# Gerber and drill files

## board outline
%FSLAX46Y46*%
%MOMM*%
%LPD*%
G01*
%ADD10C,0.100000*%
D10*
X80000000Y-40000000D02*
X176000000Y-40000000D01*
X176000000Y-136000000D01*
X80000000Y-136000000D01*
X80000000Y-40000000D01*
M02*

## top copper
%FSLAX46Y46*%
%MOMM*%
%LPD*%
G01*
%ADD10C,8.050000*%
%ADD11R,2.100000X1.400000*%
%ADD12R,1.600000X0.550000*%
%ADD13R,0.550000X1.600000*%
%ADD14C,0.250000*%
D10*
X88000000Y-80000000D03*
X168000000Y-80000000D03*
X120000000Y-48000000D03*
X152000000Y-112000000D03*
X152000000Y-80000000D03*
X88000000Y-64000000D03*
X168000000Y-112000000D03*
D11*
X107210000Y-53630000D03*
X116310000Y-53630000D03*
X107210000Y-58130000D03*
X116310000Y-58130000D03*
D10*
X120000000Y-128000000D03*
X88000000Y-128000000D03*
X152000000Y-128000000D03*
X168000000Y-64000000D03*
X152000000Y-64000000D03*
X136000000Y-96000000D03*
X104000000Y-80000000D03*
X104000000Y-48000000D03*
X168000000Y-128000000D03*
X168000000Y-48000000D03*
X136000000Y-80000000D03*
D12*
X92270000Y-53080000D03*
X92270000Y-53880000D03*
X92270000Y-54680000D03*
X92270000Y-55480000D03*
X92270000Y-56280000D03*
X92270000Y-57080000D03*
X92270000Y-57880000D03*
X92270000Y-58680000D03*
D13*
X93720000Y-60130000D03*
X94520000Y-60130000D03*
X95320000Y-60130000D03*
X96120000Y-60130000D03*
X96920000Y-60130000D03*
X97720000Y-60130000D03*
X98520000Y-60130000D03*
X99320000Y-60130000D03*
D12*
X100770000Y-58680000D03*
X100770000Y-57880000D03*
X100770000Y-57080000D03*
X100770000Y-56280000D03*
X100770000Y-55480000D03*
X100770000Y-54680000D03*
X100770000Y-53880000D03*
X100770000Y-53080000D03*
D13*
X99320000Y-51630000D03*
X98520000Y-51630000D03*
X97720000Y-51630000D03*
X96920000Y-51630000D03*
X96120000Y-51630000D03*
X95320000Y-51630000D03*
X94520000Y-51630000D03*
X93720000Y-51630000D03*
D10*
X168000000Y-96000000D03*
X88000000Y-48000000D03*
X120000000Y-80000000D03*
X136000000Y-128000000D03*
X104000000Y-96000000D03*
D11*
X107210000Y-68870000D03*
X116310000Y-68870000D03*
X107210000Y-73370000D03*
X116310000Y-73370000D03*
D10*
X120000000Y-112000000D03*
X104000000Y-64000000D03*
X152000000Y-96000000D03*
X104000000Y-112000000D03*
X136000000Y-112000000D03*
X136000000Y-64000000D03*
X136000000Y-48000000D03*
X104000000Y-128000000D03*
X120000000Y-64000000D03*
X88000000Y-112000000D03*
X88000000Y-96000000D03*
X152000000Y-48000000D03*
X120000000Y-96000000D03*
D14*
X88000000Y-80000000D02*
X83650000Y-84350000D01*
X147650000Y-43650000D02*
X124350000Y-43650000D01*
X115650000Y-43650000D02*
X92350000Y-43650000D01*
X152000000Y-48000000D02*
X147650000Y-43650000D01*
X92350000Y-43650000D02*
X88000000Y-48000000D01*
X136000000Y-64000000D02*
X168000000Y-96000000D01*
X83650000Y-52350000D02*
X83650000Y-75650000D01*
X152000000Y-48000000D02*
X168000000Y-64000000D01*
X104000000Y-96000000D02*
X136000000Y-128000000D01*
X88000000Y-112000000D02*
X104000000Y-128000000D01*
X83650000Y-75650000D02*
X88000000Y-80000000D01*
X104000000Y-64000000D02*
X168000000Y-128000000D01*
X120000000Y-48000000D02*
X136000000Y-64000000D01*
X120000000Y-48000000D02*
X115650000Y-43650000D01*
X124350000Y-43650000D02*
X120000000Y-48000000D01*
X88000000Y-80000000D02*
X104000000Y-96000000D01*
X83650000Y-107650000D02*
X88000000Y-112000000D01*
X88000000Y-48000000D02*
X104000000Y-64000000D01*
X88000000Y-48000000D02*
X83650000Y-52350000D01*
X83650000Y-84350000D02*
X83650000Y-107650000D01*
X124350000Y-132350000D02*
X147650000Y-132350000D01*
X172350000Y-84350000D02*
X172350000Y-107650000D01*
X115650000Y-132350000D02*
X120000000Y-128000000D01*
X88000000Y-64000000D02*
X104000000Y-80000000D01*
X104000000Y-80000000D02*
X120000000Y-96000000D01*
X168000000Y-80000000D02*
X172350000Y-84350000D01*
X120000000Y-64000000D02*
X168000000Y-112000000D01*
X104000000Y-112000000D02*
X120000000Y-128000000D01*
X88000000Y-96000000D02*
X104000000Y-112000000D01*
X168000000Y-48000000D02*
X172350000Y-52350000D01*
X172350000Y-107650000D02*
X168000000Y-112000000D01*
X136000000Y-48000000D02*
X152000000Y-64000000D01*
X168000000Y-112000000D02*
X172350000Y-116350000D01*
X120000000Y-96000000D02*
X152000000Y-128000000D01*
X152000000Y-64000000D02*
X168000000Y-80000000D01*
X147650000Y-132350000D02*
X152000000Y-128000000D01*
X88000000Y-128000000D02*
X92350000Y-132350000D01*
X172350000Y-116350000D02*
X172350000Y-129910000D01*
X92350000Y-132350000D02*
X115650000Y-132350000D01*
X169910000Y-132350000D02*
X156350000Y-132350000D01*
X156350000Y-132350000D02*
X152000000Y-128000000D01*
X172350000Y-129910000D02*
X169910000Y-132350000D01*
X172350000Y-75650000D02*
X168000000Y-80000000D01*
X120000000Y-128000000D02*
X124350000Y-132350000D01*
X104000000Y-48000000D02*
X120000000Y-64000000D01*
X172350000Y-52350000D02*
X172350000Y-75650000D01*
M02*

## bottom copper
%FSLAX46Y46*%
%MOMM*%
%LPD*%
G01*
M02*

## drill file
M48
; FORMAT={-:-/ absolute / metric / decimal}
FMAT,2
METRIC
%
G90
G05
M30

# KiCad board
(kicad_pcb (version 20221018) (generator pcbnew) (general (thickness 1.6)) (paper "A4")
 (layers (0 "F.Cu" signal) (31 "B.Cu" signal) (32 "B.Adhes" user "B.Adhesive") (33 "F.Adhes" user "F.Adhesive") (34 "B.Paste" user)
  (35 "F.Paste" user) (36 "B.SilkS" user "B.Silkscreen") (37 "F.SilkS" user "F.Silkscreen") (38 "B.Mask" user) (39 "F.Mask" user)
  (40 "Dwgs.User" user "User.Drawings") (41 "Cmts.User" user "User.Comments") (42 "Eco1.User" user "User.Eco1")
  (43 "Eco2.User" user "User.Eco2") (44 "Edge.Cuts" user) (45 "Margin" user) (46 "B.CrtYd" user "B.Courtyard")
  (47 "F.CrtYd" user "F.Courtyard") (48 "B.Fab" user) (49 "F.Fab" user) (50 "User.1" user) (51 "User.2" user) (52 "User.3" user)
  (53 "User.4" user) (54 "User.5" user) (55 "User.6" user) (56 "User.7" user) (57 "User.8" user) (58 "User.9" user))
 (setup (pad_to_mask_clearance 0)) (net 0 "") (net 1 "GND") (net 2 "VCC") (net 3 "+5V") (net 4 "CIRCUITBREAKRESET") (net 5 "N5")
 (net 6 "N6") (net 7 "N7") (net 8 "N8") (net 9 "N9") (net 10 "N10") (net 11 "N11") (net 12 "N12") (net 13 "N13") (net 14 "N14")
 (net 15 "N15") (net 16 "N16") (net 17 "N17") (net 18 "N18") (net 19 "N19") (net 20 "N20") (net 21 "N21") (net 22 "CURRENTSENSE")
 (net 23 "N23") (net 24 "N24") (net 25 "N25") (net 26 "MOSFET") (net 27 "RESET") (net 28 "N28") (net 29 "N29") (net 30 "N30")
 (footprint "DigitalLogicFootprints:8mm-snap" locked (layer "F.Cu") (at 88 80)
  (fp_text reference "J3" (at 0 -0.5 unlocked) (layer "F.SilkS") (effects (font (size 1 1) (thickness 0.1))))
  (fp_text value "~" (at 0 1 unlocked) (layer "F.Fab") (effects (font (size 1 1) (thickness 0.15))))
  (pad "1" smd circle locked (at 0 0) (size 8.05 8.05) (layers "F.Cu" "F.Paste" "F.Mask") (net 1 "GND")))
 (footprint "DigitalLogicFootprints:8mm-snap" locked (layer "F.Cu") (at 168 80)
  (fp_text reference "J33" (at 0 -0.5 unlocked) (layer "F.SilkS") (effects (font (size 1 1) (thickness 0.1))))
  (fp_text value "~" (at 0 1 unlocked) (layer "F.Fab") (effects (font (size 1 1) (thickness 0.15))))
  (pad "1" smd circle locked (at 0 0) (size 8.05 8.05) (layers "F.Cu" "F.Paste" "F.Mask") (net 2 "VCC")))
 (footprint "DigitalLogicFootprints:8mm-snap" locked (layer "F.Cu") (at 120 48)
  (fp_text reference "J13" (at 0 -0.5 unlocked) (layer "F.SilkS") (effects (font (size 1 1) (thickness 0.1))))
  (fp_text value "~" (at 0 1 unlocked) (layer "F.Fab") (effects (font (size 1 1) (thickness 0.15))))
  (pad "1" smd circle locked (at 0 0) (size 8.05 8.05) (layers "F.Cu" "F.Paste" "F.Mask") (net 1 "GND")))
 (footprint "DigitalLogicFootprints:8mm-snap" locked (layer "F.Cu") (at 152 112)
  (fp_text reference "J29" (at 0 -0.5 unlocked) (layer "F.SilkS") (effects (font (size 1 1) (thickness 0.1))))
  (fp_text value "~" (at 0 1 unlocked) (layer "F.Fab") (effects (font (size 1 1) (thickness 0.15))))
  (pad "1" smd circle locked (at 0 0) (size 8.05 8.05) (layers "F.Cu" "F.Paste" "F.Mask") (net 1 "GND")))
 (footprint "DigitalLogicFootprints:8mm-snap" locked (layer "F.Cu") (at 152 80)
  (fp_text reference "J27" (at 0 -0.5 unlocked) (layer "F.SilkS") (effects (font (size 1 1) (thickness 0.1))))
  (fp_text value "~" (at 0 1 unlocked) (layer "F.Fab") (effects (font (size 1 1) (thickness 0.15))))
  (pad "1" smd circle locked (at 0 0) (size 8.05 8.05) (layers "F.Cu" "F.Paste" "F.Mask") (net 1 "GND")))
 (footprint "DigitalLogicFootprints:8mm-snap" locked (layer "F.Cu") (at 88 64)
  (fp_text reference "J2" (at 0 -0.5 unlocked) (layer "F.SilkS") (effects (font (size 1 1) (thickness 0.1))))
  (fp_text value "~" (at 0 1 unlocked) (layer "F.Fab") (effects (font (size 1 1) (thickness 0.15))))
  (pad "1" smd circle locked (at 0 0) (size 8.05 8.05) (layers "F.Cu" "F.Paste" "F.Mask") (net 2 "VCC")))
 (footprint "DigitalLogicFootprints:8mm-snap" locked (layer "F.Cu") (at 168 112)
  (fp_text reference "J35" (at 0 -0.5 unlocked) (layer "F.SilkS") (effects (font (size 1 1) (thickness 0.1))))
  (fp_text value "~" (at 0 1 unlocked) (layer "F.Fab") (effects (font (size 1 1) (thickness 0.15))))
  (pad "1" smd circle locked (at 0 0) (size 8.05 8.05) (layers "F.Cu" "F.Paste" "F.Mask") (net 2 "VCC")))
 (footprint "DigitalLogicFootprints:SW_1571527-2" (layer "F.Cu") (at 111.76 55.88)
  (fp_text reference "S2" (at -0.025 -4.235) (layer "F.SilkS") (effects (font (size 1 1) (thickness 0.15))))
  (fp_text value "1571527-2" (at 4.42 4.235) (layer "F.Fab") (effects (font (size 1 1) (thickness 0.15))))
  (pad "1" smd rect (at -4.55 -2.25) (size 2.1 1.4) (layers "F.Cu" "F.Paste" "F.Mask") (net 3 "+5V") (solder_mask_margin 0.102))
  (pad "2" smd rect (at 4.55 -2.25) (size 2.1 1.4) (layers "F.Cu" "F.Paste" "F.Mask") (solder_mask_margin 0.102))
  (pad "3" smd rect (at -4.55 2.25) (size 2.1 1.4) (layers "F.Cu" "F.Paste" "F.Mask") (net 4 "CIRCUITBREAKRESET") (solder_mask_margin 0.102))
  (pad "4" smd rect (at 4.55 2.25) (size 2.1 1.4) (layers "F.Cu" "F.Paste" "F.Mask") (solder_mask_margin 0.102)))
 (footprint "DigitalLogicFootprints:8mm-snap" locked (layer "F.Cu") (at 120 128)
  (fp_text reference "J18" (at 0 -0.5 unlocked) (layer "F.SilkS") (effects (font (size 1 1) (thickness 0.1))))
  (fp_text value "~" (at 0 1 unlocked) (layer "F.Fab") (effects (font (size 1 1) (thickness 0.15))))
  (pad "1" smd circle locked (at 0 0) (size 8.05 8.05) (layers "F.Cu" "F.Paste" "F.Mask") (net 2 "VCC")))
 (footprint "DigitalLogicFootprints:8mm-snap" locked (layer "F.Cu") (at 88 128)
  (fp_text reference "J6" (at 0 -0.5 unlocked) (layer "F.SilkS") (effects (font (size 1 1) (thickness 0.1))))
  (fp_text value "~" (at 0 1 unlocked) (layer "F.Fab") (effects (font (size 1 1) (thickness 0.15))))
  (pad "1" smd circle locked (at 0 0) (size 8.05 8.05) (layers "F.Cu" "F.Paste" "F.Mask") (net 2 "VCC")))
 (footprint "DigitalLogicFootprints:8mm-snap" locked (layer "F.Cu") (at 152 128)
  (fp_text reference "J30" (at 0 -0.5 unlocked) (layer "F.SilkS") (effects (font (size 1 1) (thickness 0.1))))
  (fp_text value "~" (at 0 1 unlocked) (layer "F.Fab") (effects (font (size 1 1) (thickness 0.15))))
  (pad "1" smd circle locked (at 0 0) (size 8.05 8.05) (layers "F.Cu" "F.Paste" "F.Mask") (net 2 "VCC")))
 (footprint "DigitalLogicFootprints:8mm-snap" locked (layer "F.Cu") (at 168 64)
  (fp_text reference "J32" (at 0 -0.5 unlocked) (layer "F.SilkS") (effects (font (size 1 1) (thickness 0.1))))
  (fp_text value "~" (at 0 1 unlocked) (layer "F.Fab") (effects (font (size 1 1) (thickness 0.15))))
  (pad "1" smd circle locked (at 0 0) (size 8.05 8.05) (layers "F.Cu" "F.Paste" "F.Mask") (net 1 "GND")))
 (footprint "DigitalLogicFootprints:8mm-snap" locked (layer "F.Cu") (at 152 64)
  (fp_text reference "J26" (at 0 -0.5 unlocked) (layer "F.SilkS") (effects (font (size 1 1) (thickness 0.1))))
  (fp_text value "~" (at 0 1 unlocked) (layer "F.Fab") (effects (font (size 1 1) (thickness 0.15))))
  (pad "1" smd circle locked (at 0 0) (size 8.05 8.05) (layers "F.Cu" "F.Paste" "F.Mask") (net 2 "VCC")))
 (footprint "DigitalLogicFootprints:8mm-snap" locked (layer "F.Cu") (at 136 96)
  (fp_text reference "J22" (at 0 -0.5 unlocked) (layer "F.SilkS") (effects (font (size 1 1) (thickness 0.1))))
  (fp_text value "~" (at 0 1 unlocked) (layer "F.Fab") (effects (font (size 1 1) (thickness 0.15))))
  (pad "1" smd circle locked (at 0 0) (size 8.05 8.05) (layers "F.Cu" "F.Paste" "F.Mask") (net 1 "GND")))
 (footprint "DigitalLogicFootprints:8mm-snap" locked (layer "F.Cu") (at 104 80)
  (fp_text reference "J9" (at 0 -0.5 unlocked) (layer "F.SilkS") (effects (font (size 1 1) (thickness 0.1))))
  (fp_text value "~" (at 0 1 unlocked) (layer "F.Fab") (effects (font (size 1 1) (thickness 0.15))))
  (pad "1" smd circle locked (at 0 0) (size 8.05 8.05) (layers "F.Cu" "F.Paste" "F.Mask") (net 2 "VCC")))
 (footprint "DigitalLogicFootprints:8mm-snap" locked (layer "F.Cu") (at 104 48)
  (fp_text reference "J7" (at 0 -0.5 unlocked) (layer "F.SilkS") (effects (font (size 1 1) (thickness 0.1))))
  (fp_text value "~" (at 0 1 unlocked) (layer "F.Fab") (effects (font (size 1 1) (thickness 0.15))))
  (pad "1" smd circle locked (at 0 0) (size 8.05 8.05) (layers "F.Cu" "F.Paste" "F.Mask") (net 2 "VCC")))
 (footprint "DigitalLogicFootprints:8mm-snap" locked (layer "F.Cu") (at 168 128)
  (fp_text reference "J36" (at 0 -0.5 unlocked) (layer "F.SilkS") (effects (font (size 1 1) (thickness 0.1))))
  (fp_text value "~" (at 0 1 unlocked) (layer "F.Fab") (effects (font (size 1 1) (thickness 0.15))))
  (pad "1" smd circle locked (at 0 0) (size 8.05 8.05) (layers "F.Cu" "F.Paste" "F.Mask") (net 1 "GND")))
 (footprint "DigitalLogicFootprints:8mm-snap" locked (layer "F.Cu") (at 168 48)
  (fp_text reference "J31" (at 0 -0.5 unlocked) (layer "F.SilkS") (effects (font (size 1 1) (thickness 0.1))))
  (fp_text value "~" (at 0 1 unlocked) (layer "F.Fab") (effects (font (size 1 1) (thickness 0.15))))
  (pad "1" smd circle locked (at 0 0) (size 8.05 8.05) (layers "F.Cu" "F.Paste" "F.Mask") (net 2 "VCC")))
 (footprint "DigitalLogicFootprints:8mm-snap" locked (layer "F.Cu") (at 136 80)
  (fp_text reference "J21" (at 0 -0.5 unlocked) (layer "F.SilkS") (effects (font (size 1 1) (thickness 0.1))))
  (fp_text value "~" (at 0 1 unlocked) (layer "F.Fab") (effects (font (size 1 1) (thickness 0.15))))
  (pad "1" smd circle locked (at 0 0) (size 8.05 8.05) (layers "F.Cu" "F.Paste" "F.Mask") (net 2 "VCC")))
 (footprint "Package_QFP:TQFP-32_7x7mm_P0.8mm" (layer "F.Cu") (at 96.52 55.88)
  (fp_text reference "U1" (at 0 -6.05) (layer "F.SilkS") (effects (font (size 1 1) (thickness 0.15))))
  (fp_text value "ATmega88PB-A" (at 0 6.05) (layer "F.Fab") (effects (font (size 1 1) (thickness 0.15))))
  (pad "1" smd rect (at -4.25 -2.8) (size 1.6 0.55) (layers "F.Cu" "F.Paste" "F.Mask") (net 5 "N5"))
  (pad "2" smd rect (at -4.25 -2) (size 1.6 0.55) (layers "F.Cu" "F.Paste" "F.Mask") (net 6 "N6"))
  (pad "3" smd rect (at -4.25 -1.2) (size 1.6 0.55) (layers "F.Cu" "F.Paste" "F.Mask") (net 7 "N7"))
  (pad "4" smd rect (at -4.25 -0.4) (size 1.6 0.55) (layers "F.Cu" "F.Paste" "F.Mask") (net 3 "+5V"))
  (pad "5" smd rect (at -4.25 0.4) (size 1.6 0.55) (layers "F.Cu" "F.Paste" "F.Mask") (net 1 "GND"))
  (pad "6" smd rect (at -4.25 1.2) (size 1.6 0.55) (layers "F.Cu" "F.Paste" "F.Mask") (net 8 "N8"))
  (pad "7" smd rect (at -4.25 2) (size 1.6 0.55) (layers "F.Cu" "F.Paste" "F.Mask") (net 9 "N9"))
  (pad "8" smd rect (at -4.25 2.8) (size 1.6 0.55) (layers "F.Cu" "F.Paste" "F.Mask") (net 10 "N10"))
  (pad "9" smd rect (at -2.8 4.25 90) (size 1.6 0.55) (layers "F.Cu" "F.Paste" "F.Mask") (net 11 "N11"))
  (pad "10" smd rect (at -2 4.25 90) (size 1.6 0.55) (layers "F.Cu" "F.Paste" "F.Mask") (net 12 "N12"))
  (pad "11" smd rect (at -1.2 4.25 90) (size 1.6 0.55) (layers "F.Cu" "F.Paste" "F.Mask") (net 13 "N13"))
  (pad "12" smd rect (at -0.4 4.25 90) (size 1.6 0.55) (layers "F.Cu" "F.Paste" "F.Mask") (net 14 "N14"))
  (pad "13" smd rect (at 0.4 4.25 90) (size 1.6 0.55) (layers "F.Cu" "F.Paste" "F.Mask") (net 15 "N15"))
  (pad "14" smd rect (at 1.2 4.25 90) (size 1.6 0.55) (layers "F.Cu" "F.Paste" "F.Mask") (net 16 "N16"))
  (pad "15" smd rect (at 2 4.25 90) (size 1.6 0.55) (layers "F.Cu" "F.Paste" "F.Mask") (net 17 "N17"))
  (pad "16" smd rect (at 2.8 4.25 90) (size 1.6 0.55) (layers "F.Cu" "F.Paste" "F.Mask") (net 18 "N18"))
  (pad "17" smd rect (at 4.25 2.8) (size 1.6 0.55) (layers "F.Cu" "F.Paste" "F.Mask") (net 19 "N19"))
  (pad "18" smd rect (at 4.25 2) (size 1.6 0.55) (layers "F.Cu" "F.Paste" "F.Mask") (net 3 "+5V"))
  (pad "19" smd rect (at 4.25 1.2) (size 1.6 0.55) (layers "F.Cu" "F.Paste" "F.Mask") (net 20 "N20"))
  (pad "20" smd rect (at 4.25 0.4) (size 1.6 0.55) (layers "F.Cu" "F.Paste" "F.Mask") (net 3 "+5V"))
  (pad "21" smd rect (at 4.25 -0.4) (size 1.6 0.55) (layers "F.Cu" "F.Paste" "F.Mask") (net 1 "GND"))
  (pad "22" smd rect (at 4.25 -1.2) (size 1.6 0.55) (layers "F.Cu" "F.Paste" "F.Mask") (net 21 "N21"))
  (pad "23" smd rect (at 4.25 -2) (size 1.6 0.55) (layers "F.Cu" "F.Paste" "F.Mask") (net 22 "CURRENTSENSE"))
  (pad "24" smd rect (at 4.25 -2.8) (size 1.6 0.55) (layers "F.Cu" "F.Paste" "F.Mask") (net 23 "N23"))
  (pad "25" smd rect (at 2.8 -4.25 90) (size 1.6 0.55) (layers "F.Cu" "F.Paste" "F.Mask") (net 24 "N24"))
  (pad "26" smd rect (at 2 -4.25 90) (size 1.6 0.55) (layers "F.Cu" "F.Paste" "F.Mask") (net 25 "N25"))
  (pad "27" smd rect (at 1.2 -4.25 90) (size 1.6 0.55) (layers "F.Cu" "F.Paste" "F.Mask") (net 4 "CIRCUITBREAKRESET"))
  (pad "28" smd rect (at 0.4 -4.25 90) (size 1.6 0.55) (layers "F.Cu" "F.Paste" "F.Mask") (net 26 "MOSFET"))
  (pad "29" smd rect (at -0.4 -4.25 90) (size 1.6 0.55) (layers "F.Cu" "F.Paste" "F.Mask") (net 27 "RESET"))
  (pad "30" smd rect (at -1.2 -4.25 90) (size 1.6 0.55) (layers "F.Cu" "F.Paste" "F.Mask") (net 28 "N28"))
  (pad "31" smd rect (at -2 -4.25 90) (size 1.6 0.55) (layers "F.Cu" "F.Paste" "F.Mask") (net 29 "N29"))
  (pad "32" smd rect (at -2.8 -4.25 90) (size 1.6 0.55) (layers "F.Cu" "F.Paste" "F.Mask") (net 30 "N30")))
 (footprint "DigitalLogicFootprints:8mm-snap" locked (layer "F.Cu") (at 168 96)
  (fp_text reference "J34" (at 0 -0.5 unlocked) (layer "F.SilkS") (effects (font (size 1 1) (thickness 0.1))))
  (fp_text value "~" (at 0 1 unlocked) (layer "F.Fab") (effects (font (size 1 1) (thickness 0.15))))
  (pad "1" smd circle locked (at 0 0) (size 8.05 8.05) (layers "F.Cu" "F.Paste" "F.Mask") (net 1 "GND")))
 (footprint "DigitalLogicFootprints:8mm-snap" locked (layer "F.Cu") (at 88 48)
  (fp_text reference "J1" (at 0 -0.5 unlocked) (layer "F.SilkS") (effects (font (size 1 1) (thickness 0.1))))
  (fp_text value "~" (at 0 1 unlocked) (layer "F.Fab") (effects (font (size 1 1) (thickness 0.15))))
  (pad "1" smd circle locked (at 0 0) (size 8.05 8.05) (layers "F.Cu" "F.Paste" "F.Mask") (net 1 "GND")))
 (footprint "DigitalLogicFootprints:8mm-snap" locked (layer "F.Cu") (at 120 80)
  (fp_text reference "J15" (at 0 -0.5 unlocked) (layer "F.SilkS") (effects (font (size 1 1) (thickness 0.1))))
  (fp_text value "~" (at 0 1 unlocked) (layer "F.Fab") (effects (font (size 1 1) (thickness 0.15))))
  (pad "1" smd circle locked (at 0 0) (size 8.05 8.05) (layers "F.Cu" "F.Paste" "F.Mask") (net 1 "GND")))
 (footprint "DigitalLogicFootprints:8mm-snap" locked (layer "F.Cu") (at 136 128)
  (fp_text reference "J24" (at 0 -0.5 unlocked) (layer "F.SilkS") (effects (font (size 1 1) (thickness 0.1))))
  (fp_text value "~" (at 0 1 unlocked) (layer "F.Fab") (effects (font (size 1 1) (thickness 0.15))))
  (pad "1" smd circle locked (at 0 0) (size 8.05 8.05) (layers "F.Cu" "F.Paste" "F.Mask") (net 1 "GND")))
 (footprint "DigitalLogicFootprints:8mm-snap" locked (layer "F.Cu") (at 104 96)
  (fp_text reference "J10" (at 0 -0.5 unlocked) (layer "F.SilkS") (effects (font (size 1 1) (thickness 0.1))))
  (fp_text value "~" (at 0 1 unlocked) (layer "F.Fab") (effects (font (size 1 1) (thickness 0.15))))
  (pad "1" smd circle locked (at 0 0) (size 8.05 8.05) (layers "F.Cu" "F.Paste" "F.Mask") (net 1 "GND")))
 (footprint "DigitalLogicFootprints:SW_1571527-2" (layer "F.Cu") (at 111.76 71.12)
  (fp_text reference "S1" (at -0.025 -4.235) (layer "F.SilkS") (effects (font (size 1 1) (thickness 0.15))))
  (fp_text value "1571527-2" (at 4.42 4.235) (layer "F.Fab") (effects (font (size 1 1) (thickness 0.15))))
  (pad "1" smd rect (at -4.55 -2.25) (size 2.1 1.4) (layers "F.Cu" "F.Paste" "F.Mask") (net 3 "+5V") (solder_mask_margin 0.102))
  (pad "2" smd rect (at 4.55 -2.25) (size 2.1 1.4) (layers "F.Cu" "F.Paste" "F.Mask") (solder_mask_margin 0.102))
  (pad "3" smd rect (at -4.55 2.25) (size 2.1 1.4) (layers "F.Cu" "F.Paste" "F.Mask") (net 27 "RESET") (solder_mask_margin 0.102))
  (pad "4" smd rect (at 4.55 2.25) (size 2.1 1.4) (layers "F.Cu" "F.Paste" "F.Mask") (solder_mask_margin 0.102)))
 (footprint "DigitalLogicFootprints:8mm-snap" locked (layer "F.Cu") (at 120 112)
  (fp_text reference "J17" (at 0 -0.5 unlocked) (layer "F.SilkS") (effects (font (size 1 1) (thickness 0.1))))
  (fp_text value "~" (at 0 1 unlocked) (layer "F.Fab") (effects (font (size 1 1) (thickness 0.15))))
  (pad "1" smd circle locked (at 0 0) (size 8.05 8.05) (layers "F.Cu" "F.Paste" "F.Mask") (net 1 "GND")))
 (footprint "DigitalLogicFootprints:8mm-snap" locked (layer "F.Cu") (at 104 64)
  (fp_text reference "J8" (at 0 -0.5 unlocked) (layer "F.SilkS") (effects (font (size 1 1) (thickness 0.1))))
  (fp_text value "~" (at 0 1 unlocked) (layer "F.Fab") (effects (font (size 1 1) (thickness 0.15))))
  (pad "1" smd circle locked (at 0 0) (size 8.05 8.05) (layers "F.Cu" "F.Paste" "F.Mask") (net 1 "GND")))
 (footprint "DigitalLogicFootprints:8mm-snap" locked (layer "F.Cu") (at 152 96)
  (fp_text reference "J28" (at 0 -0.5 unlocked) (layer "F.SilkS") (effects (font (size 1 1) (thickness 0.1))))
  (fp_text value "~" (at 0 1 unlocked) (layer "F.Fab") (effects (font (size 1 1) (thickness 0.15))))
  (pad "1" smd circle locked (at 0 0) (size 8.05 8.05) (layers "F.Cu" "F.Paste" "F.Mask") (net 2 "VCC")))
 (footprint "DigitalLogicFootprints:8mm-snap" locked (layer "F.Cu") (at 104 112)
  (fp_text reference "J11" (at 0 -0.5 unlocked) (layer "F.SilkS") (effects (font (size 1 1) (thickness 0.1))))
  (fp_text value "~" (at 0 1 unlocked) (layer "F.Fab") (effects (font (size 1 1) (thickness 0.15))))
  (pad "1" smd circle locked (at 0 0) (size 8.05 8.05) (layers "F.Cu" "F.Paste" "F.Mask") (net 2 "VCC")))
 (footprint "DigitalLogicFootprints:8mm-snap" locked (layer "F.Cu") (at 136 112)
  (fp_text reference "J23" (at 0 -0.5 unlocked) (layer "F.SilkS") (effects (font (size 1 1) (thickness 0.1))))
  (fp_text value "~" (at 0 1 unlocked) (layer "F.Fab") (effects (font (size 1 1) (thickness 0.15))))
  (pad "1" smd circle locked (at 0 0) (size 8.05 8.05) (layers "F.Cu" "F.Paste" "F.Mask") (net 2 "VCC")))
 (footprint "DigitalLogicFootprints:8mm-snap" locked (layer "F.Cu") (at 136 64)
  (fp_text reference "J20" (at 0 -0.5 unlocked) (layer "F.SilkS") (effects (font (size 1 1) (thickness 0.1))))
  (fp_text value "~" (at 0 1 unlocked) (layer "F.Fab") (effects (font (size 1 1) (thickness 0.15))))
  (pad "1" smd circle locked (at 0 0) (size 8.05 8.05) (layers "F.Cu" "F.Paste" "F.Mask") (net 1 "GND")))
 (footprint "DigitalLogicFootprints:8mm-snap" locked (layer "F.Cu") (at 136 48)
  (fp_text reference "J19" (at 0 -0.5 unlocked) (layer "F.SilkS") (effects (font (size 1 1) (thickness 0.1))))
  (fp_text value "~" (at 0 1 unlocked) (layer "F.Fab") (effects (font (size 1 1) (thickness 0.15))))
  (pad "1" smd circle locked (at 0 0) (size 8.05 8.05) (layers "F.Cu" "F.Paste" "F.Mask") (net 2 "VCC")))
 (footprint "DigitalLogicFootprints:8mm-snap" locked (layer "F.Cu") (at 104 128)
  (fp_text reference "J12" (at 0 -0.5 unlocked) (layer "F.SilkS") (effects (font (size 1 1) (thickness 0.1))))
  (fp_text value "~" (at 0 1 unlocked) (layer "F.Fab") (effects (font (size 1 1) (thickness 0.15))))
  (pad "1" smd circle locked (at 0 0) (size 8.05 8.05) (layers "F.Cu" "F.Paste" "F.Mask") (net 1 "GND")))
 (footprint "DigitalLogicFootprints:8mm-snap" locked (layer "F.Cu") (at 120 64)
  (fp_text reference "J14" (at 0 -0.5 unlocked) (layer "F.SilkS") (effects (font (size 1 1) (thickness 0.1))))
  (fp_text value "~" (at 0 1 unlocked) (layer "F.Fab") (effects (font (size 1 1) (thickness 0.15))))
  (pad "1" smd circle locked (at 0 0) (size 8.05 8.05) (layers "F.Cu" "F.Paste" "F.Mask") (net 2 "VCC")))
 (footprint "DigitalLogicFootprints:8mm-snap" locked (layer "F.Cu") (at 88 112)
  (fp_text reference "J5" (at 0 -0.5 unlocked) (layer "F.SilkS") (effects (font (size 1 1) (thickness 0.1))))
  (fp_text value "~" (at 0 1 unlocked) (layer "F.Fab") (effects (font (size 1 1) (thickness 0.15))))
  (pad "1" smd circle locked (at 0 0) (size 8.05 8.05) (layers "F.Cu" "F.Paste" "F.Mask") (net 1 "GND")))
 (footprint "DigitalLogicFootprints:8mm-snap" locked (layer "F.Cu") (at 88 96)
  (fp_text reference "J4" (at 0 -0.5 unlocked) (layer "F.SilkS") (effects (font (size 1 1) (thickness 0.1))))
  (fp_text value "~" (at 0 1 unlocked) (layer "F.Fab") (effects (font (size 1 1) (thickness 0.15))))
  (pad "1" smd circle locked (at 0 0) (size 8.05 8.05) (layers "F.Cu" "F.Paste" "F.Mask") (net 2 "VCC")))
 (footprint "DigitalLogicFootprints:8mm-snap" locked (layer "F.Cu") (at 152 48)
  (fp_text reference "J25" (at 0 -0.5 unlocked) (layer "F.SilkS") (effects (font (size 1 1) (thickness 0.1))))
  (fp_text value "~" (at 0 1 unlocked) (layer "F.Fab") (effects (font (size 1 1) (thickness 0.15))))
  (pad "1" smd circle locked (at 0 0) (size 8.05 8.05) (layers "F.Cu" "F.Paste" "F.Mask") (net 1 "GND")))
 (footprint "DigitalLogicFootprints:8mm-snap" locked (layer "F.Cu") (at 120 96)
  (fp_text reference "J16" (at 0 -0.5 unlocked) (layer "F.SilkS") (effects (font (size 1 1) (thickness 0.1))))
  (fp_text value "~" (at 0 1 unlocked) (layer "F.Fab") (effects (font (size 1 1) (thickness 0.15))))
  (pad "1" smd circle locked (at 0 0) (size 8.05 8.05) (layers "F.Cu" "F.Paste" "F.Mask") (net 2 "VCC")))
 (gr_rect (start 80 40) (end 176 136) (stroke (width 0.1) (type default)) (fill none) (layer "Edge.Cuts"))
 (segment (start 88 80) (end 83.65 84.35) (width 0.25) (layer "F.Cu") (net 1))
 (segment (start 147.65 43.65) (end 124.35 43.65) (width 0.25) (layer "F.Cu") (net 1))
 (segment (start 115.65 43.65) (end 92.35 43.65) (width 0.25) (layer "F.Cu") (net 1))
 (segment (start 152 48) (end 147.65 43.65) (width 0.25) (layer "F.Cu") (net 1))
 (segment (start 92.35 43.65) (end 88 48) (width 0.25) (layer "F.Cu") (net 1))
 (segment (start 136 64) (end 168 96) (width 0.25) (layer "F.Cu") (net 1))
 (segment (start 83.65 52.35) (end 83.65 75.65) (width 0.25) (layer "F.Cu") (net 1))
 (segment (start 152 48) (end 168 64) (width 0.25) (layer "F.Cu") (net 1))
 (segment (start 104 96) (end 136 128) (width 0.25) (layer "F.Cu") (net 1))
 (segment (start 88 112) (end 104 128) (width 0.25) (layer "F.Cu") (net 1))
 (segment (start 83.65 75.65) (end 88 80) (width 0.25) (layer "F.Cu") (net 1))
 (segment (start 104 64) (end 168 128) (width 0.25) (layer "F.Cu") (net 1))
 (segment (start 120 48) (end 136 64) (width 0.25) (layer "F.Cu") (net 1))
 (segment (start 120 48) (end 115.65 43.65) (width 0.25) (layer "F.Cu") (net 1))
 (segment (start 124.35 43.65) (end 120 48) (width 0.25) (layer "F.Cu") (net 1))
 (segment (start 88 80) (end 104 96) (width 0.25) (layer "F.Cu") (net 1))
 (segment (start 83.65 107.65) (end 88 112) (width 0.25) (layer "F.Cu") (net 1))
 (segment (start 88 48) (end 104 64) (width 0.25) (layer "F.Cu") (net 1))
 (segment (start 88 48) (end 83.65 52.35) (width 0.25) (layer "F.Cu") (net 1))
 (segment (start 83.65 84.35) (end 83.65 107.65) (width 0.25) (layer "F.Cu") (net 1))
 (segment (start 124.35 132.35) (end 147.65 132.35) (width 0.25) (layer "F.Cu") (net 2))
 (segment (start 172.35 84.35) (end 172.35 107.65) (width 0.25) (layer "F.Cu") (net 2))
 (segment (start 115.65 132.35) (end 120 128) (width 0.25) (layer "F.Cu") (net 2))
 (segment (start 88 64) (end 104 80) (width 0.25) (layer "F.Cu") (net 2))
 (segment (start 104 80) (end 120 96) (width 0.25) (layer "F.Cu") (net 2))
 (segment (start 168 80) (end 172.35 84.35) (width 0.25) (layer "F.Cu") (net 2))
 (segment (start 120 64) (end 168 112) (width 0.25) (layer "F.Cu") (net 2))
 (segment (start 104 112) (end 120 128) (width 0.25) (layer "F.Cu") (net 2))
 (segment (start 88 96) (end 104 112) (width 0.25) (layer "F.Cu") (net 2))
 (segment (start 168 48) (end 172.35 52.35) (width 0.25) (layer "F.Cu") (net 2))
 (segment (start 172.35 107.65) (end 168 112) (width 0.25) (layer "F.Cu") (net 2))
 (segment (start 136 48) (end 152 64) (width 0.25) (layer "F.Cu") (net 2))
 (segment (start 168 112) (end 172.35 116.35) (width 0.25) (layer "F.Cu") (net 2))
 (segment (start 120 96) (end 152 128) (width 0.25) (layer "F.Cu") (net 2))
 (segment (start 152 64) (end 168 80) (width 0.25) (layer "F.Cu") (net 2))
 (segment (start 147.65 132.35) (end 152 128) (width 0.25) (layer "F.Cu") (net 2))
 (segment (start 88 128) (end 92.35 132.35) (width 0.25) (layer "F.Cu") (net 2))
 (segment (start 172.35 116.35) (end 172.35 129.91) (width 0.25) (layer "F.Cu") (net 2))
 (segment (start 92.35 132.35) (end 115.65 132.35) (width 0.25) (layer "F.Cu") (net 2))
 (segment (start 169.91 132.35) (end 156.35 132.35) (width 0.25) (layer "F.Cu") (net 2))
 (segment (start 156.35 132.35) (end 152 128) (width 0.25) (layer "F.Cu") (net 2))
 (segment (start 172.35 129.91) (end 169.91 132.35) (width 0.25) (layer "F.Cu") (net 2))
 (segment (start 172.35 75.65) (end 168 80) (width 0.25) (layer "F.Cu") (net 2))
 (segment (start 120 128) (end 124.35 132.35) (width 0.25) (layer "F.Cu") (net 2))
 (segment (start 104 48) (end 120 64) (width 0.25) (layer "F.Cu") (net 2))
 (segment (start 172.35 52.35) (end 172.35 75.65) (width 0.25) (layer "F.Cu") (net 2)))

